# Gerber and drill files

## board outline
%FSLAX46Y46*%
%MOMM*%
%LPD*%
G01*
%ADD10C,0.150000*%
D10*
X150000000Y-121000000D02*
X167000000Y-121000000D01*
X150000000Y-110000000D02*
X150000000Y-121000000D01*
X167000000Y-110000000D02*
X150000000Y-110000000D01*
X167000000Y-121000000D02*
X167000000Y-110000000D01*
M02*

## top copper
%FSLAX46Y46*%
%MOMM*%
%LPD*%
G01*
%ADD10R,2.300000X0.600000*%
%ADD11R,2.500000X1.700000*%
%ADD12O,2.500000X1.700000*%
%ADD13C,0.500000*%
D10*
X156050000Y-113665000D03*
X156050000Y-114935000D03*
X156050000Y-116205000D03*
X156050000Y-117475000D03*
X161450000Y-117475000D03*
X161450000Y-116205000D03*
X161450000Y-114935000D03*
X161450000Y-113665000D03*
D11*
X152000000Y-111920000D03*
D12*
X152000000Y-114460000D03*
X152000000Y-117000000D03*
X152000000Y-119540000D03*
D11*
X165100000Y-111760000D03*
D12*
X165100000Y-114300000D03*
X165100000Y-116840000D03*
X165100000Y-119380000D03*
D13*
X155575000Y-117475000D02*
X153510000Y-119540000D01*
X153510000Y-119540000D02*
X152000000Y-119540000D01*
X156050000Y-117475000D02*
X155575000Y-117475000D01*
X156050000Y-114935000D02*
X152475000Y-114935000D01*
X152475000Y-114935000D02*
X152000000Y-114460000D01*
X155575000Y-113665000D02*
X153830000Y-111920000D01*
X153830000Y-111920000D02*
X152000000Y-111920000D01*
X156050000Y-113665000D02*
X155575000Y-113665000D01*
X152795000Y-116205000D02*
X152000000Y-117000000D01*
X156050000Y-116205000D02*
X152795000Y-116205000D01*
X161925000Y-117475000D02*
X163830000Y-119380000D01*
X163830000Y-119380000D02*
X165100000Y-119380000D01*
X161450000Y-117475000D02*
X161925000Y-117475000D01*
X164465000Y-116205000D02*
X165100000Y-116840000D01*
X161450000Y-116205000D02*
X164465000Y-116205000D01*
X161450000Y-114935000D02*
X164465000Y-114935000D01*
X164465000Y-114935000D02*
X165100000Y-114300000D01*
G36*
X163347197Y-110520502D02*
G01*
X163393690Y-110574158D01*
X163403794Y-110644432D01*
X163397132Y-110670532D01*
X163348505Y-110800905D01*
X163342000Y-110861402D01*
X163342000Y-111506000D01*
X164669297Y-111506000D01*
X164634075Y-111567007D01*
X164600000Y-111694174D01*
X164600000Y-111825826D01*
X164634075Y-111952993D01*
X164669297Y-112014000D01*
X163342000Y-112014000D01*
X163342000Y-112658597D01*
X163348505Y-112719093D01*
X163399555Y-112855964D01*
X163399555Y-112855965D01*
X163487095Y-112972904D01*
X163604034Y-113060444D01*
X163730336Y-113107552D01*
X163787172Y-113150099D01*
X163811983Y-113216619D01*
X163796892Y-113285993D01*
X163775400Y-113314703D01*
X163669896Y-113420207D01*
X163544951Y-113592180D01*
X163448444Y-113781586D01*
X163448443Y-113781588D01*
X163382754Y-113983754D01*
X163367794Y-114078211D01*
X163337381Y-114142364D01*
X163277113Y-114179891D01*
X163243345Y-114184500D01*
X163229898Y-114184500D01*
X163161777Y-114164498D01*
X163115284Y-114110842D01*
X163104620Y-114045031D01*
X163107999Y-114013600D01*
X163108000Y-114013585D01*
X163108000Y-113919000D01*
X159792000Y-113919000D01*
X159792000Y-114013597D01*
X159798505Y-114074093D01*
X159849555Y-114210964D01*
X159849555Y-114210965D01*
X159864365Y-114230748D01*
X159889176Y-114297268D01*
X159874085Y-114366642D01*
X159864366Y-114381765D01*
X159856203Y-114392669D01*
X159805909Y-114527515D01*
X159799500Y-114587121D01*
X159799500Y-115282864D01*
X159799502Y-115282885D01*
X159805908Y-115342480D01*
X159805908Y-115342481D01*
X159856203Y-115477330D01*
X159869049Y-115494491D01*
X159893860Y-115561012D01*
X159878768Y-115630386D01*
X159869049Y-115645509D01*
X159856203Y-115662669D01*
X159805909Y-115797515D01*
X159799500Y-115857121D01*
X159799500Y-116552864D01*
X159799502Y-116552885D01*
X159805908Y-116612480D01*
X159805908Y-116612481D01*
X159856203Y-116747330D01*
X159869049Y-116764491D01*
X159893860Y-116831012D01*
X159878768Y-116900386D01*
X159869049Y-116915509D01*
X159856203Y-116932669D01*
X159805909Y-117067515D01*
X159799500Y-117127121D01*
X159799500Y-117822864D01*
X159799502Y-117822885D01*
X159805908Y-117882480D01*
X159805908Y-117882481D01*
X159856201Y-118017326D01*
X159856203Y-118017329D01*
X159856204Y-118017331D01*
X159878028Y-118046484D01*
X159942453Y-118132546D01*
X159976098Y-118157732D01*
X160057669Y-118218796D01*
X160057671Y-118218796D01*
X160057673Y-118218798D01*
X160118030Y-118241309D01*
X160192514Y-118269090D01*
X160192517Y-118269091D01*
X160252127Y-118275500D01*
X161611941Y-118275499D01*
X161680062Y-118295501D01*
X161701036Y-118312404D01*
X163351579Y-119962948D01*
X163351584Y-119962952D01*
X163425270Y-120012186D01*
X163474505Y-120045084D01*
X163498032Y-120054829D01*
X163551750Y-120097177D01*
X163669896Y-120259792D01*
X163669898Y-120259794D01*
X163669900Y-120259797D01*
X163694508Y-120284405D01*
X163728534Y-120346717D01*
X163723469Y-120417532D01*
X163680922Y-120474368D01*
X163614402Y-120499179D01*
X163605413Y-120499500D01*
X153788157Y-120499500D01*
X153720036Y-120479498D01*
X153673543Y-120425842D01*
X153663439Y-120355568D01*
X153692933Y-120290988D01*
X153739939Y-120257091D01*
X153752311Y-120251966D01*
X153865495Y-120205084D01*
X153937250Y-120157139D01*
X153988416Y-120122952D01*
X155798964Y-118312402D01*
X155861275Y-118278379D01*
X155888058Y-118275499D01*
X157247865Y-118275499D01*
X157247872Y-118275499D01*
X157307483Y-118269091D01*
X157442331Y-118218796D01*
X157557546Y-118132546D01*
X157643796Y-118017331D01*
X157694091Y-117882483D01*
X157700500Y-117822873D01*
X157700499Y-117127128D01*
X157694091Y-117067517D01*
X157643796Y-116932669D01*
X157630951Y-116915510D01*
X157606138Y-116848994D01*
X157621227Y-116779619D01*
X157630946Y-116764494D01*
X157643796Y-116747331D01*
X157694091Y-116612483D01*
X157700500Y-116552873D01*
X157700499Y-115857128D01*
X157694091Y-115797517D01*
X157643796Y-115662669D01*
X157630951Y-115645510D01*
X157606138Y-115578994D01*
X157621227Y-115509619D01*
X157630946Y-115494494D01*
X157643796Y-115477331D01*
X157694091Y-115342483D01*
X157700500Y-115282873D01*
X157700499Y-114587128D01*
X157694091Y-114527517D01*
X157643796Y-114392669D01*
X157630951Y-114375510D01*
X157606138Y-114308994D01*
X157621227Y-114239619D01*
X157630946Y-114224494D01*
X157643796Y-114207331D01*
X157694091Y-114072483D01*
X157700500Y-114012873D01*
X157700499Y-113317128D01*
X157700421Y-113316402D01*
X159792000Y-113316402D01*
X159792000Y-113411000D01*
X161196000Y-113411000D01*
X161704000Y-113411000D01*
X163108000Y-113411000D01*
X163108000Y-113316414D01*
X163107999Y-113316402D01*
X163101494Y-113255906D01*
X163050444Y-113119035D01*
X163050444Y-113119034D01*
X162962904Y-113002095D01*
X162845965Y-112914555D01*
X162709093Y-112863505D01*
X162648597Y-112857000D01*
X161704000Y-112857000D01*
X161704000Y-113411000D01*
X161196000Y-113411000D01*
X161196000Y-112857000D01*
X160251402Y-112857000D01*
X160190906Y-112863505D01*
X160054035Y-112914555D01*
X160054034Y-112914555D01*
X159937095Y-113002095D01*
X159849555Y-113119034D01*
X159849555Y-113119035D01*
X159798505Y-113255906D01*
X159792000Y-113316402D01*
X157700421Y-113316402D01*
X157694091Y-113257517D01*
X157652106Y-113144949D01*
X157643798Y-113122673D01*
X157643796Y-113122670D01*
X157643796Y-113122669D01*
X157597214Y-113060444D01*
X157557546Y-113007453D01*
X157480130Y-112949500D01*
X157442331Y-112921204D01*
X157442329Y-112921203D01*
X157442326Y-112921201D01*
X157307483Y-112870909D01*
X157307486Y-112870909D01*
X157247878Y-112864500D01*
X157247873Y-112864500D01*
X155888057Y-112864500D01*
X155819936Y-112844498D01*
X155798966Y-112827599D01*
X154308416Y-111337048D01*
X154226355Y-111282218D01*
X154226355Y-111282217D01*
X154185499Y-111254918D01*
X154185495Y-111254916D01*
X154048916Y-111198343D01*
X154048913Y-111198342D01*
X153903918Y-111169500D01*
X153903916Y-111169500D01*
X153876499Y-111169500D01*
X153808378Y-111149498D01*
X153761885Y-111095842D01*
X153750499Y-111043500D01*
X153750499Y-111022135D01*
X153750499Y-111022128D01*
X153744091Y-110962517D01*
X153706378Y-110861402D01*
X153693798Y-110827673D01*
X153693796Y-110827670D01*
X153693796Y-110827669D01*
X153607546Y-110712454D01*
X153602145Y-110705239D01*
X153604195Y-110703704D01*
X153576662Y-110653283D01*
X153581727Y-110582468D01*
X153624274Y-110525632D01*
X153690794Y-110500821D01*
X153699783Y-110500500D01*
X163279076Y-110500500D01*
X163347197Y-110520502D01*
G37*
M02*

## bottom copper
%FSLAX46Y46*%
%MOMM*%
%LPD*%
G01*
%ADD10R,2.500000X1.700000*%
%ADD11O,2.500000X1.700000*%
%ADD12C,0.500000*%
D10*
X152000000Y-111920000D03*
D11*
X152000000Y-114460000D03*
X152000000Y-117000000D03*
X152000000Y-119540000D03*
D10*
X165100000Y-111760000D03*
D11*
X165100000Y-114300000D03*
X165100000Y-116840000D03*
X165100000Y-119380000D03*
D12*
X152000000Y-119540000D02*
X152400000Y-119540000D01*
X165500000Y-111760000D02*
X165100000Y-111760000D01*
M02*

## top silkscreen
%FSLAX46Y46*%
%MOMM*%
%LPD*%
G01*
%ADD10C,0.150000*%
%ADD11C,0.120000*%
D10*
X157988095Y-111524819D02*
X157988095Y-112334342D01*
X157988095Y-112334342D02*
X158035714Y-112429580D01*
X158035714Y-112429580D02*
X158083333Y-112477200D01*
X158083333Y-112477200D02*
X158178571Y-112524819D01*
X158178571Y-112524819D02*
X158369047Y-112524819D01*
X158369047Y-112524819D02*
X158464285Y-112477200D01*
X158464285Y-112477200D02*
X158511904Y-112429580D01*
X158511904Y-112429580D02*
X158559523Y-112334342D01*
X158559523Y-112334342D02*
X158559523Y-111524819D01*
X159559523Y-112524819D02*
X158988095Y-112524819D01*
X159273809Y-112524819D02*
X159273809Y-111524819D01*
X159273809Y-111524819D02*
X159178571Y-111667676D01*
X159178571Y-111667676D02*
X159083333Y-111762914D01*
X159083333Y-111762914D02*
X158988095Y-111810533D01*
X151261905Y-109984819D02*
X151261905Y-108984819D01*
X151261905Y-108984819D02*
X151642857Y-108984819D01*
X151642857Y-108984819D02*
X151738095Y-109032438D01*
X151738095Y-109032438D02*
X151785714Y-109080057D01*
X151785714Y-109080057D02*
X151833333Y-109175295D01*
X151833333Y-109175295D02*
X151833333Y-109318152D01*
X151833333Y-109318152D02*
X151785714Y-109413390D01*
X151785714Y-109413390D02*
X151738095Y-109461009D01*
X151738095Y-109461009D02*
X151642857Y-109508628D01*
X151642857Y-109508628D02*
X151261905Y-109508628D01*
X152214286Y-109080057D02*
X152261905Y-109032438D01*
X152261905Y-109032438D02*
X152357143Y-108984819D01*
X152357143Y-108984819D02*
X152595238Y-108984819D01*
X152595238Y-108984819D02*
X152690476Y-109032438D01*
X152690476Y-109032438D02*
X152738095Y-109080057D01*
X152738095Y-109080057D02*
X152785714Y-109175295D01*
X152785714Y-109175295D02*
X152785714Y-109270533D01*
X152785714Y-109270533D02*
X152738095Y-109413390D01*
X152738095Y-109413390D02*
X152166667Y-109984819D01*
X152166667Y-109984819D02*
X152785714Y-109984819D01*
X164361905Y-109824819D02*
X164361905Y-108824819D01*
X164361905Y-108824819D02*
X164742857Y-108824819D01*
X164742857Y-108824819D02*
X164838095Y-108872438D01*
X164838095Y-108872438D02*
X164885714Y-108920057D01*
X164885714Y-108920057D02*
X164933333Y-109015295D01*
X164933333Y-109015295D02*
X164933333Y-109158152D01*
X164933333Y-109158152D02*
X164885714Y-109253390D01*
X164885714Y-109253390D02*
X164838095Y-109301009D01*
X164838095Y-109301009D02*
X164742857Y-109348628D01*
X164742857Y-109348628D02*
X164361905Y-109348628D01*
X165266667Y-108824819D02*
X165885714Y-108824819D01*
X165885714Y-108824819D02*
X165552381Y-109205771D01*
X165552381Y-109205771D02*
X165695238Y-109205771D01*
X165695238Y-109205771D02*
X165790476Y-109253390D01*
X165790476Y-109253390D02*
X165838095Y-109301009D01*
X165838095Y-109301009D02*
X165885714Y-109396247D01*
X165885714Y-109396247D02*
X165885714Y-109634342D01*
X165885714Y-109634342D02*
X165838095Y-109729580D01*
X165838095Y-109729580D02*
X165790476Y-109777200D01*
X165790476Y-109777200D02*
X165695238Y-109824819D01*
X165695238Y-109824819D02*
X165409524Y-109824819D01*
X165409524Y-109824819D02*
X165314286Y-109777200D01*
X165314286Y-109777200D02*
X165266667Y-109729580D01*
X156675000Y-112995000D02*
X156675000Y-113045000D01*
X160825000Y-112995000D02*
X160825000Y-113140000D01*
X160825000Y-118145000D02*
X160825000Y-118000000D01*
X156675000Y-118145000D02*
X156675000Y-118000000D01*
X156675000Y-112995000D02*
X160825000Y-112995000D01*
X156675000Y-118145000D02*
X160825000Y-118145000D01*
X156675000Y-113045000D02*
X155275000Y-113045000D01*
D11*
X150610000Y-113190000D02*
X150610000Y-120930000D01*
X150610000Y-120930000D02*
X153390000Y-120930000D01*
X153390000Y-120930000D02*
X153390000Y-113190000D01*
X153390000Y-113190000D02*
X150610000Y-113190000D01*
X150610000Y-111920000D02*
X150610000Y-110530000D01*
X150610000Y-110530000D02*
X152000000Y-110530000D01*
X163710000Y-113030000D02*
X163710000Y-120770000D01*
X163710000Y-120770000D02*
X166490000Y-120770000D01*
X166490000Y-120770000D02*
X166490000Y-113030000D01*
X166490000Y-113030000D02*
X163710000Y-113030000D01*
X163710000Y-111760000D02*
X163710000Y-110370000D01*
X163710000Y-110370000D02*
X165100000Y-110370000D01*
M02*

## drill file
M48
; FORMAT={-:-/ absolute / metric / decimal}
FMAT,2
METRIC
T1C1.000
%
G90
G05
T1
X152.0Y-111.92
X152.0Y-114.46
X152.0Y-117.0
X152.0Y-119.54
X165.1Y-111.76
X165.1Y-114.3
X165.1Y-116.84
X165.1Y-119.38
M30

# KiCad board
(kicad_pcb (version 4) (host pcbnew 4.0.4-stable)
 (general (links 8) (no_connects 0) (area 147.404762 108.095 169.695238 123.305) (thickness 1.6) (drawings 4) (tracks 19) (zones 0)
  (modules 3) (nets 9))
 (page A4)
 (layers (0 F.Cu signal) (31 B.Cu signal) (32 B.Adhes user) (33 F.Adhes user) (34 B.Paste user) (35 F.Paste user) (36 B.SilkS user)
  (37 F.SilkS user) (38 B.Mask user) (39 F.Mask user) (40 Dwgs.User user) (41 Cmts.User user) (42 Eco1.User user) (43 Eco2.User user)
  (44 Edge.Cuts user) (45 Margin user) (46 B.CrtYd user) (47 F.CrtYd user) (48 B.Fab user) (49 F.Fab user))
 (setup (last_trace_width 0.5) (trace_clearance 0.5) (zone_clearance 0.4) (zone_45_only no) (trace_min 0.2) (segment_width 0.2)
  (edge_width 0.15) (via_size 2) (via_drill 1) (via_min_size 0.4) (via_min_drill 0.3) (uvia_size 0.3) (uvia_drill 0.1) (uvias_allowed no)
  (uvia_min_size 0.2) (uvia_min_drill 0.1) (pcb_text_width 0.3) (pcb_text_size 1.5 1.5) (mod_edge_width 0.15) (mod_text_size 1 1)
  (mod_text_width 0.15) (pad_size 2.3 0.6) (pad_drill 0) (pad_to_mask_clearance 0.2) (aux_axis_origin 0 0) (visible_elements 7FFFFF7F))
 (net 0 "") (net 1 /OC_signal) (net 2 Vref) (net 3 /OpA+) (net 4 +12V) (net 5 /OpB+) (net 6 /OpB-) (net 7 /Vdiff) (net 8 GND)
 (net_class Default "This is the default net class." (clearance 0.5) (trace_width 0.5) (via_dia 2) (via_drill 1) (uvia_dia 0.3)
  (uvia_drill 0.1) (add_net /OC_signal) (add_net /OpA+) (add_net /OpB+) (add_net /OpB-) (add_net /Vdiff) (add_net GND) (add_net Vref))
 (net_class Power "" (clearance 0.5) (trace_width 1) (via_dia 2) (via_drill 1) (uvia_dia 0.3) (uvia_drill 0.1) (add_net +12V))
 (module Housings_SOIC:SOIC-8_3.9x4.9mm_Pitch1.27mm (layer F.Cu) (at 158.75 115.57)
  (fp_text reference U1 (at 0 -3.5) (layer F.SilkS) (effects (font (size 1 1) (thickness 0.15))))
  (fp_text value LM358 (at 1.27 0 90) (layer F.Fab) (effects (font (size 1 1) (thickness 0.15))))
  (fp_line (start -2.075 -2.575) (end -2.075 -2.525) (layer F.SilkS) (width 0.15))
  (fp_line (start 2.075 -2.575) (end 2.075 -2.43) (layer F.SilkS) (width 0.15))
  (fp_line (start 2.075 2.575) (end 2.075 2.43) (layer F.SilkS) (width 0.15))
  (fp_line (start -2.075 2.575) (end -2.075 2.43) (layer F.SilkS) (width 0.15))
  (fp_line (start -2.075 -2.575) (end 2.075 -2.575) (layer F.SilkS) (width 0.15))
  (fp_line (start -2.075 2.575) (end 2.075 2.575) (layer F.SilkS) (width 0.15))
  (fp_line (start -2.075 -2.525) (end -3.475 -2.525) (layer F.SilkS) (width 0.15))
  (pad 1 smd rect (at -2.7 -1.905) (size 2.3 0.6) (layers F.Cu F.Paste F.Mask) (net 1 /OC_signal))
  (pad 2 smd rect (at -2.7 -0.635) (size 2.3 0.6) (layers F.Cu F.Paste F.Mask) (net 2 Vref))
  (pad 3 smd rect (at -2.7 0.635) (size 2.3 0.6) (layers F.Cu F.Paste F.Mask) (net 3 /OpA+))
  (pad 4 smd rect (at -2.7 1.905) (size 2.3 0.6) (layers F.Cu F.Paste F.Mask) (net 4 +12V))
  (pad 5 smd rect (at 2.7 1.905) (size 2.3 0.6) (layers F.Cu F.Paste F.Mask) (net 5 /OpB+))
  (pad 6 smd rect (at 2.7 0.635) (size 2.3 0.6) (layers F.Cu F.Paste F.Mask) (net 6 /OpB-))
  (pad 7 smd rect (at 2.7 -0.635) (size 2.3 0.6) (layers F.Cu F.Paste F.Mask) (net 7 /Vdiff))
  (pad 8 smd rect (at 2.7 -1.905) (size 2.3 0.6) (layers F.Cu F.Paste F.Mask) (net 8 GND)))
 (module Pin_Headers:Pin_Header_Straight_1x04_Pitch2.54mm (layer F.Cu) (at 152 111.92)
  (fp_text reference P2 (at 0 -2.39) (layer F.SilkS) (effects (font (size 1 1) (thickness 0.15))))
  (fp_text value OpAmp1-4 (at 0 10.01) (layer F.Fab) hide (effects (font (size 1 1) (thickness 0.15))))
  (fp_line (start -1.39 1.27) (end -1.39 9.01) (layer F.SilkS) (width 0.12))
  (fp_line (start -1.39 9.01) (end 1.39 9.01) (layer F.SilkS) (width 0.12))
  (fp_line (start 1.39 9.01) (end 1.39 1.27) (layer F.SilkS) (width 0.12))
  (fp_line (start 1.39 1.27) (end -1.39 1.27) (layer F.SilkS) (width 0.12))
  (fp_line (start -1.39 0) (end -1.39 -1.39) (layer F.SilkS) (width 0.12))
  (fp_line (start -1.39 -1.39) (end 0 -1.39) (layer F.SilkS) (width 0.12))
  (pad 1 thru_hole rect (at 0 0) (size 2.5 1.7) (drill 1) (layers *.Cu *.Mask) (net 1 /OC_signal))
  (pad 2 thru_hole oval (at 0 2.54) (size 2.5 1.7) (drill 1) (layers *.Cu *.Mask) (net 2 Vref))
  (pad 3 thru_hole oval (at 0 5.08) (size 2.5 1.7) (drill 1) (layers *.Cu *.Mask) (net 3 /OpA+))
  (pad 4 thru_hole oval (at 0 7.62) (size 2.5 1.7) (drill 1) (layers *.Cu *.Mask) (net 4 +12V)))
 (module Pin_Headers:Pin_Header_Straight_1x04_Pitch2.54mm (layer F.Cu) (at 165.1 111.76)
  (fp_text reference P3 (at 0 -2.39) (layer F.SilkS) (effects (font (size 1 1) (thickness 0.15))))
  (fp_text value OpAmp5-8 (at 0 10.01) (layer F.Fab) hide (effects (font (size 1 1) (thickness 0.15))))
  (fp_line (start -1.39 1.27) (end -1.39 9.01) (layer F.SilkS) (width 0.12))
  (fp_line (start -1.39 9.01) (end 1.39 9.01) (layer F.SilkS) (width 0.12))
  (fp_line (start 1.39 9.01) (end 1.39 1.27) (layer F.SilkS) (width 0.12))
  (fp_line (start 1.39 1.27) (end -1.39 1.27) (layer F.SilkS) (width 0.12))
  (fp_line (start -1.39 0) (end -1.39 -1.39) (layer F.SilkS) (width 0.12))
  (fp_line (start -1.39 -1.39) (end 0 -1.39) (layer F.SilkS) (width 0.12))
  (pad 1 thru_hole rect (at 0 0) (size 2.5 1.7) (drill 1) (layers *.Cu *.Mask) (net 8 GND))
  (pad 2 thru_hole oval (at 0 2.54) (size 2.5 1.7) (drill 1) (layers *.Cu *.Mask) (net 7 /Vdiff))
  (pad 3 thru_hole oval (at 0 5.08) (size 2.5 1.7) (drill 1) (layers *.Cu *.Mask) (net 6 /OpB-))
  (pad 4 thru_hole oval (at 0 7.62) (size 2.5 1.7) (drill 1) (layers *.Cu *.Mask) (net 5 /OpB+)))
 (gr_line (start 150 121) (end 167 121) (layer Edge.Cuts) (width 0.15))
 (gr_line (start 150 110) (end 150 121) (layer Edge.Cuts) (width 0.15))
 (gr_line (start 167 110) (end 150 110) (layer Edge.Cuts) (width 0.15))
 (gr_line (start 167 121) (end 167 110) (layer Edge.Cuts) (width 0.15))
 (segment (start 152 119.54) (end 152.4 119.54) (width 0.5) (layer B.Cu) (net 4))
 (segment (start 155.575 117.475) (end 153.51 119.54) (width 0.5) (layer F.Cu) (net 4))
 (segment (start 153.51 119.54) (end 152 119.54) (width 0.5) (layer F.Cu) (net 4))
 (segment (start 156.05 117.475) (end 155.575 117.475) (width 0.5) (layer F.Cu) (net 4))
 (segment (start 156.05 114.935) (end 152.475 114.935) (width 0.5) (layer F.Cu) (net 2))
 (segment (start 152.475 114.935) (end 152 114.46) (width 0.5) (layer F.Cu) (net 2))
 (segment (start 165.5 111.76) (end 165.1 111.76) (width 0.5) (layer B.Cu) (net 8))
 (segment (start 155.575 113.665) (end 153.83 111.92) (width 0.5) (layer F.Cu) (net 1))
 (segment (start 153.83 111.92) (end 152 111.92) (width 0.5) (layer F.Cu) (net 1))
 (segment (start 156.05 113.665) (end 155.575 113.665) (width 0.5) (layer F.Cu) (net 1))
 (segment (start 152.795 116.205) (end 152 117) (width 0.5) (layer F.Cu) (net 3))
 (segment (start 156.05 116.205) (end 152.795 116.205) (width 0.5) (layer F.Cu) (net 3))
 (segment (start 161.925 117.475) (end 163.83 119.38) (width 0.5) (layer F.Cu) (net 5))
 (segment (start 163.83 119.38) (end 165.1 119.38) (width 0.5) (layer F.Cu) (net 5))
 (segment (start 161.45 117.475) (end 161.925 117.475) (width 0.5) (layer F.Cu) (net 5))
 (segment (start 164.465 116.205) (end 165.1 116.84) (width 0.5) (layer F.Cu) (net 6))
 (segment (start 161.45 116.205) (end 164.465 116.205) (width 0.5) (layer F.Cu) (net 6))
 (segment (start 161.45 114.935) (end 164.465 114.935) (width 0.5) (layer F.Cu) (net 7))
 (segment (start 164.465 114.935) (end 165.1 114.3) (width 0.5) (layer F.Cu) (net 7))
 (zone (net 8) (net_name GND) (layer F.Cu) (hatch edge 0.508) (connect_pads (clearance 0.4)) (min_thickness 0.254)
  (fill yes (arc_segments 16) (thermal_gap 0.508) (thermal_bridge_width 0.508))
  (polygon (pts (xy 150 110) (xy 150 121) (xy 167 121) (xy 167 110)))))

